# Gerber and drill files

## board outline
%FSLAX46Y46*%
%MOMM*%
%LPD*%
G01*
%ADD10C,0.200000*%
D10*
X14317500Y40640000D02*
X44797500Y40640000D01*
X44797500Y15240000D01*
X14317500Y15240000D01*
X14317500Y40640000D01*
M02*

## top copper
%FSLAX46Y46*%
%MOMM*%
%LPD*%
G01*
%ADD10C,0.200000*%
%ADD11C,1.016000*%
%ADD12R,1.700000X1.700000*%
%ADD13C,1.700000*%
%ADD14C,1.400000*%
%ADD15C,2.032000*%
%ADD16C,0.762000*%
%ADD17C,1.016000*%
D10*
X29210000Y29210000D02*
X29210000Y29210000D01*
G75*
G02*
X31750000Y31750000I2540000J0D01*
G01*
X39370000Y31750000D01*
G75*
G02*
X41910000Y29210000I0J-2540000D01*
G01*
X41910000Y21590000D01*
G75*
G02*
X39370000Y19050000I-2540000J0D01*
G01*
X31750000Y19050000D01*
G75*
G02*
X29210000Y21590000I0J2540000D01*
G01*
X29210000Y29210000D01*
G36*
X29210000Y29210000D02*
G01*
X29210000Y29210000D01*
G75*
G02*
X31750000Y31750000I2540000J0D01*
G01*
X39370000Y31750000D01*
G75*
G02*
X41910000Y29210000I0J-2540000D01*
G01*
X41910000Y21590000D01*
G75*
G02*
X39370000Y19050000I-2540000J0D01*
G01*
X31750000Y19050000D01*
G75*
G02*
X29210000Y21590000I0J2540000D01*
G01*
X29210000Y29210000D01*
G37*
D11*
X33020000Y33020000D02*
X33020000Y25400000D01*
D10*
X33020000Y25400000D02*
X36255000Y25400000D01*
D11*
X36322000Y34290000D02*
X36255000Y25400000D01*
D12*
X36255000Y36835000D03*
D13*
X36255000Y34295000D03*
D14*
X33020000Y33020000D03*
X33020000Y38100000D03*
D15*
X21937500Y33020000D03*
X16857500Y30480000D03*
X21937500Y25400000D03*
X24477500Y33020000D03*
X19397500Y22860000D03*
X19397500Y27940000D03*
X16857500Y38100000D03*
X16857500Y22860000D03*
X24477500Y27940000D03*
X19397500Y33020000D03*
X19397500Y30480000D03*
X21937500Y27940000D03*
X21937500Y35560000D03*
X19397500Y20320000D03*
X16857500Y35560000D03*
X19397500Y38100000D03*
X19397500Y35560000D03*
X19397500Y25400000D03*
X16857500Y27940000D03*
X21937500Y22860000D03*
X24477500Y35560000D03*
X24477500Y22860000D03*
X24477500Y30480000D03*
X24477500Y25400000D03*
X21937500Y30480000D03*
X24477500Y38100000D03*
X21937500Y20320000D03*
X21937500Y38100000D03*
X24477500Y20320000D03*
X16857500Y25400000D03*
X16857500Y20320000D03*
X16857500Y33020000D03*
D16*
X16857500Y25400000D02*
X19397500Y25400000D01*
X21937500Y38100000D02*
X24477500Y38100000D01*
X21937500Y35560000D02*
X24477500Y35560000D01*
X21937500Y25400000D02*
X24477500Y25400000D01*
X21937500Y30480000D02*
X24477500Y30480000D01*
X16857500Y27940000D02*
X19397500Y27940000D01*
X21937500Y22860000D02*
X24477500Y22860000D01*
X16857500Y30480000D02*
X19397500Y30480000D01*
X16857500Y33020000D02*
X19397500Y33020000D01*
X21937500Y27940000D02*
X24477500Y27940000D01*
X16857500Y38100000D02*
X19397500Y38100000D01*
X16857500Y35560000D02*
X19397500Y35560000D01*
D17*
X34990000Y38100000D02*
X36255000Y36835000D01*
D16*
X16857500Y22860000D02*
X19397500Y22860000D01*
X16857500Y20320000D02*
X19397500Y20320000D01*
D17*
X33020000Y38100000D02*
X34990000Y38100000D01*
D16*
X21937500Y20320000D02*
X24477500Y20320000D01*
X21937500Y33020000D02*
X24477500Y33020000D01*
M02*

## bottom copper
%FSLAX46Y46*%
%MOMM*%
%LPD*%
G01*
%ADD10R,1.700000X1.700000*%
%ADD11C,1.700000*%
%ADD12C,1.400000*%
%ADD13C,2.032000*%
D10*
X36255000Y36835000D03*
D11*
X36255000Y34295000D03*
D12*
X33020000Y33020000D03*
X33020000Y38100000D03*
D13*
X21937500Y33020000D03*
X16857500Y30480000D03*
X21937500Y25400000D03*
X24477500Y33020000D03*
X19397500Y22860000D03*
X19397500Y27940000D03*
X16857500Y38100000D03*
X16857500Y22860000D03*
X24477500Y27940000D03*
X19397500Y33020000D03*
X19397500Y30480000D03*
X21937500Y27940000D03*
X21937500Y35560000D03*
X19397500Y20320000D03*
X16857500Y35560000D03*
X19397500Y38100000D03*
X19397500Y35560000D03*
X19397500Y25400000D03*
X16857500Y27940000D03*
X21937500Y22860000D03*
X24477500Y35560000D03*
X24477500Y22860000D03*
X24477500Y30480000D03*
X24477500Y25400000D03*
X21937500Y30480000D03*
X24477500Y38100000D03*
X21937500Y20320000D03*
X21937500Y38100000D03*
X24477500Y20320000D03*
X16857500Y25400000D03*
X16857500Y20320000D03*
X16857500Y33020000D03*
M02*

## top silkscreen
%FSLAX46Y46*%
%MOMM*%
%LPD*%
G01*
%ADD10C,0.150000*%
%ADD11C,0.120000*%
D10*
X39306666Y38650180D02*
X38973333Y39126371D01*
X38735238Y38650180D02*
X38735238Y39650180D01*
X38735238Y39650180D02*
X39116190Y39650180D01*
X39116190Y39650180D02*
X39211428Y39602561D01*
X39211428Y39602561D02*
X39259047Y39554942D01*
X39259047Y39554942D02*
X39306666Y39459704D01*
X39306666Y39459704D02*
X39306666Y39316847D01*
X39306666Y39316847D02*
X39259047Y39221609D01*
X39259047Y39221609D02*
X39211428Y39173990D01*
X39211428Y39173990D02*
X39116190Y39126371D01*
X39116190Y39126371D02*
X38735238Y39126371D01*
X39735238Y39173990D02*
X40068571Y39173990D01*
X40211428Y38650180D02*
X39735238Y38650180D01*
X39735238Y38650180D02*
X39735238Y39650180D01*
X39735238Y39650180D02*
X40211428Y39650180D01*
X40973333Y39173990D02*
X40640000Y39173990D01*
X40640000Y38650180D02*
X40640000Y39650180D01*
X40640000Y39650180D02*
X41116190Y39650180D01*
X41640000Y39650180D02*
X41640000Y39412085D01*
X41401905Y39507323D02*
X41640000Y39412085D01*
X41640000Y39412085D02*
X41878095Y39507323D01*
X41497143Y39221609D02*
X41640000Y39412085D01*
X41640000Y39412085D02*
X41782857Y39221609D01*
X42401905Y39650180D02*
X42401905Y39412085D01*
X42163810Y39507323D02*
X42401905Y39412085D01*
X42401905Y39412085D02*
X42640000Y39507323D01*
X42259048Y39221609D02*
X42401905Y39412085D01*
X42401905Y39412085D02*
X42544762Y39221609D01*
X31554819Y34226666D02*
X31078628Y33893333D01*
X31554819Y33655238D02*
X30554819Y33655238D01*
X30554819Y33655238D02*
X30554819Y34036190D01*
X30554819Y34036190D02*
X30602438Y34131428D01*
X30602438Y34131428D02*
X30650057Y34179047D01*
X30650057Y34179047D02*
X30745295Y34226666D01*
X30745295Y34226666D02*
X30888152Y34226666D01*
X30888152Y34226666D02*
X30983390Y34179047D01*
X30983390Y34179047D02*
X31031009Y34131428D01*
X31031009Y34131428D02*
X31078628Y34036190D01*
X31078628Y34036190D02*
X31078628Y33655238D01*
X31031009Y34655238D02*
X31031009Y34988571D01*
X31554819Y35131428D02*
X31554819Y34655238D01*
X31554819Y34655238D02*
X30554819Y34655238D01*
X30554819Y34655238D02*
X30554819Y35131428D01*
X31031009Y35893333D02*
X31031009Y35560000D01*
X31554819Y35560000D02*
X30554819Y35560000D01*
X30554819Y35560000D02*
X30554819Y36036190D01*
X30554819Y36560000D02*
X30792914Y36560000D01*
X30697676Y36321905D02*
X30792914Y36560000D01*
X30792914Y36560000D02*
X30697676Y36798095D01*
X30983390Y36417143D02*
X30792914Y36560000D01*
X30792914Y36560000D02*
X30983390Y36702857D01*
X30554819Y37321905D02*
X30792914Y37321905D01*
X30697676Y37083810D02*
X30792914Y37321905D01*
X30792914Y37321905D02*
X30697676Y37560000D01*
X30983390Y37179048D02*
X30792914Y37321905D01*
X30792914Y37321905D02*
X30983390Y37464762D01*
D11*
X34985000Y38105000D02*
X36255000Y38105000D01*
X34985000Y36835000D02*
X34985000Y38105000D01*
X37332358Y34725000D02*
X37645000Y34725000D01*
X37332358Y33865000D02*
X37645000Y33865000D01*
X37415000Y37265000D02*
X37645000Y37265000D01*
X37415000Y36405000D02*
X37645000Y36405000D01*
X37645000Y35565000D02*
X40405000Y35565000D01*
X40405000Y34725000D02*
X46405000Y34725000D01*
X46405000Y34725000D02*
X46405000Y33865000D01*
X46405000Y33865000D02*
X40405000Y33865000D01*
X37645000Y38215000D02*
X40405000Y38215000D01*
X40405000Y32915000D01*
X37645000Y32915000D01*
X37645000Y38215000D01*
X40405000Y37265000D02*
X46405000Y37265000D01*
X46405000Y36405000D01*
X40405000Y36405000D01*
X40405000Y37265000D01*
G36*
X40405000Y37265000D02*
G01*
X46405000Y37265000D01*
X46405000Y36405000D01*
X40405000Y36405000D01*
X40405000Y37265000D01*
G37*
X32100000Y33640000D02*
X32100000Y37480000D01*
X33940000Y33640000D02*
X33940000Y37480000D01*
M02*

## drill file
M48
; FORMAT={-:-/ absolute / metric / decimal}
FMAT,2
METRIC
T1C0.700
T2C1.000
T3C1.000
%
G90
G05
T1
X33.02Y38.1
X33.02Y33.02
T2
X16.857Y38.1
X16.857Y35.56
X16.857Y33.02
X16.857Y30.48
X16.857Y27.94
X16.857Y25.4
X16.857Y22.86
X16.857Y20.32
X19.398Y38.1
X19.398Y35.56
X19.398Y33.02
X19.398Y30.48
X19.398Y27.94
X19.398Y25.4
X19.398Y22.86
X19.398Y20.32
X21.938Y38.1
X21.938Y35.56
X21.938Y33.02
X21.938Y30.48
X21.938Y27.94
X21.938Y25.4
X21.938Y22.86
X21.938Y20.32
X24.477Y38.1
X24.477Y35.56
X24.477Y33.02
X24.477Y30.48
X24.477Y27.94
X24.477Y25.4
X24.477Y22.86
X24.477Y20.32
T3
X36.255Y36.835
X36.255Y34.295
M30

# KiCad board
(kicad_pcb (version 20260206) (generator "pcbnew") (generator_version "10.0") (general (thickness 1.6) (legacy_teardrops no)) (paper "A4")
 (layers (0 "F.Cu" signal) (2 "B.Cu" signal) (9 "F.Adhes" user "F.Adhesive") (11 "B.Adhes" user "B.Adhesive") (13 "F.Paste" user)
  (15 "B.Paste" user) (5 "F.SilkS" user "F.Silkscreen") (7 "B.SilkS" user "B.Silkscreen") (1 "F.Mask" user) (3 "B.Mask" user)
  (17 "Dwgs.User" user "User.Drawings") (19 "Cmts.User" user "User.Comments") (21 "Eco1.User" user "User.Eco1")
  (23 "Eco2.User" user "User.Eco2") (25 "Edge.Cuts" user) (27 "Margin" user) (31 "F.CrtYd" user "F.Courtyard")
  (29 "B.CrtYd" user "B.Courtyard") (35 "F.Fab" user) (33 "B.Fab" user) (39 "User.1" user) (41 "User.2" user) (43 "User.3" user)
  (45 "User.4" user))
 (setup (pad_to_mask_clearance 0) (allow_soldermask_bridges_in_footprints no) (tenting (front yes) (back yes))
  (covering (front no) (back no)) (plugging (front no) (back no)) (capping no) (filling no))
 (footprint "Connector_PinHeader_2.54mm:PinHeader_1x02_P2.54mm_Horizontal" (layer "F.Cu") (at 36.255 -36.835)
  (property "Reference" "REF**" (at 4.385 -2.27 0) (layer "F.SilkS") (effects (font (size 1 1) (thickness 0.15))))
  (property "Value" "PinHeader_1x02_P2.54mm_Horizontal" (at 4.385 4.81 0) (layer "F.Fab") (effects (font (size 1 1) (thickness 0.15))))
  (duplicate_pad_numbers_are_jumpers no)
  (fp_line (start -1.27 -1.27) (end 0 -1.27) (stroke (width 0.12) (type solid)) (layer "F.SilkS"))
  (fp_line (start -1.27 0) (end -1.27 -1.27) (stroke (width 0.12) (type solid)) (layer "F.SilkS"))
  (fp_line (start 1.077358 2.11) (end 1.39 2.11) (stroke (width 0.12) (type solid)) (layer "F.SilkS"))
  (fp_line (start 1.077358 2.97) (end 1.39 2.97) (stroke (width 0.12) (type solid)) (layer "F.SilkS"))
  (fp_line (start 1.16 -0.43) (end 1.39 -0.43) (stroke (width 0.12) (type solid)) (layer "F.SilkS"))
  (fp_line (start 1.16 0.43) (end 1.39 0.43) (stroke (width 0.12) (type solid)) (layer "F.SilkS"))
  (fp_line (start 1.39 1.27) (end 4.15 1.27) (stroke (width 0.12) (type solid)) (layer "F.SilkS"))
  (fp_line (start 4.15 2.11) (end 10.15 2.11) (stroke (width 0.12) (type solid)) (layer "F.SilkS"))
  (fp_line (start 10.15 2.11) (end 10.15 2.97) (stroke (width 0.12) (type solid)) (layer "F.SilkS"))
  (fp_line (start 10.15 2.97) (end 4.15 2.97) (stroke (width 0.12) (type solid)) (layer "F.SilkS"))
  (fp_rect (start 1.39 -1.38) (end 4.15 3.92) (stroke (width 0.12) (type solid)) (fill no) (layer "F.SilkS"))
  (fp_rect (start 4.15 -0.43) (end 10.15 0.43) (stroke (width 0.12) (type solid)) (fill yes) (layer "F.SilkS"))
  (pad "1" thru_hole rect (at 0 0) (size 1.7 1.7) (drill 1) (layers "*.Cu" "*.Mask") (remove_unused_layers no))
  (pad "2" thru_hole circle (at 0 2.54) (size 1.7 1.7) (drill 1) (layers "*.Cu" "*.Mask") (remove_unused_layers no)))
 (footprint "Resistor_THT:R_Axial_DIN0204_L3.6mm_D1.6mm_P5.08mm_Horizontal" (layer "F.Cu") (at 33.02 -33.02 90)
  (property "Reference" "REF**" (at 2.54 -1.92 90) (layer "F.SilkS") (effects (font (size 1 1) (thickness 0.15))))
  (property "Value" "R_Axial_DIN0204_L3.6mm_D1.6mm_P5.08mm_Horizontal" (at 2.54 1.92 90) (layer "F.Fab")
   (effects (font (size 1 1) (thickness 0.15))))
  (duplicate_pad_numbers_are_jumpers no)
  (fp_line (start 0.62 -0.92) (end 4.46 -0.92) (stroke (width 0.12) (type solid)) (layer "F.SilkS"))
  (fp_line (start 0.62 0.92) (end 4.46 0.92) (stroke (width 0.12) (type solid)) (layer "F.SilkS"))
  (pad "1" thru_hole circle (at 0 0 90) (size 1.4 1.4) (drill 0.7) (layers "*.Cu" "*.Mask") (remove_unused_layers no))
  (pad "2" thru_hole circle (at 5.08 0 90) (size 1.4 1.4) (drill 0.7) (layers "*.Cu" "*.Mask") (remove_unused_layers no)))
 (gr_rect (start 29.21 -31.75) (end 41.91 -19.05) (radius 2.54) (stroke (width 0.2) (type default)) (fill yes) (layer "F.Cu"))
 (gr_line (start 33.02 -33.02) (end 33.02 -25.4) (stroke (width 1.016) (type default)) (layer "F.Cu"))
 (gr_line (start 33.02 -25.4) (end 36.255 -25.4) (stroke (width 0.2) (type default)) (layer "F.Cu"))
 (gr_line (start 36.322 -34.29) (end 36.255 -25.4) (stroke (width 1.016) (type default)) (layer "F.Cu"))
 (gr_rect (start 14.3175 -40.64) (end 44.7975 -15.24) (stroke (width 0.2) (type default)) (fill no) (layer "Edge.Cuts"))
 (segment (start 16.8575 -25.4) (end 19.3975 -25.4) (width 0.762) (layer "F.Cu") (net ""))
 (segment (start 21.9375 -38.1) (end 24.4775 -38.1) (width 0.762) (layer "F.Cu") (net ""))
 (segment (start 21.9375 -35.56) (end 24.4775 -35.56) (width 0.762) (layer "F.Cu") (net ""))
 (segment (start 21.9375 -25.4) (end 24.4775 -25.4) (width 0.762) (layer "F.Cu") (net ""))
 (segment (start 21.9375 -30.48) (end 24.4775 -30.48) (width 0.762) (layer "F.Cu") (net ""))
 (segment (start 16.8575 -27.94) (end 19.3975 -27.94) (width 0.762) (layer "F.Cu") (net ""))
 (segment (start 21.9375 -22.86) (end 24.4775 -22.86) (width 0.762) (layer "F.Cu") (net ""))
 (segment (start 16.8575 -30.48) (end 19.3975 -30.48) (width 0.762) (layer "F.Cu") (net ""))
 (segment (start 16.8575 -33.02) (end 19.3975 -33.02) (width 0.762) (layer "F.Cu") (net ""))
 (segment (start 21.9375 -27.94) (end 24.4775 -27.94) (width 0.762) (layer "F.Cu") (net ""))
 (segment (start 16.8575 -38.1) (end 19.3975 -38.1) (width 0.762) (layer "F.Cu") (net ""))
 (segment (start 16.8575 -35.56) (end 19.3975 -35.56) (width 0.762) (layer "F.Cu") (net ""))
 (segment (start 34.99 -38.1) (end 36.255 -36.835) (width 1.016) (layer "F.Cu") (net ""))
 (segment (start 16.8575 -22.86) (end 19.3975 -22.86) (width 0.762) (layer "F.Cu") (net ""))
 (segment (start 16.8575 -20.32) (end 19.3975 -20.32) (width 0.762) (layer "F.Cu") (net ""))
 (segment (start 33.02 -38.1) (end 34.99 -38.1) (width 1.016) (layer "F.Cu") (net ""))
 (segment (start 21.9375 -20.32) (end 24.4775 -20.32) (width 0.762) (layer "F.Cu") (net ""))
 (segment (start 21.9375 -33.02) (end 24.4775 -33.02) (width 0.762) (layer "F.Cu") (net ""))
 (via (at 21.9375 -33.02) (size 2.032) (drill 1) (layers "F.Cu" "B.Cu") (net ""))
 (via (at 16.8575 -30.48) (size 2.032) (drill 1) (layers "F.Cu" "B.Cu") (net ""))
 (via (at 21.9375 -25.4) (size 2.032) (drill 1) (layers "F.Cu" "B.Cu") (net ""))
 (via (at 24.4775 -33.02) (size 2.032) (drill 1) (layers "F.Cu" "B.Cu") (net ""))
 (via (at 19.3975 -22.86) (size 2.032) (drill 1) (layers "F.Cu" "B.Cu") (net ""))
 (via (at 19.3975 -27.94) (size 2.032) (drill 1) (layers "F.Cu" "B.Cu") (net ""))
 (via (at 16.8575 -38.1) (size 2.032) (drill 1) (layers "F.Cu" "B.Cu") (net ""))
 (via (at 16.8575 -22.86) (size 2.032) (drill 1) (layers "F.Cu" "B.Cu") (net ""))
 (via (at 24.4775 -27.94) (size 2.032) (drill 1) (layers "F.Cu" "B.Cu") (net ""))
 (via (at 19.3975 -33.02) (size 2.032) (drill 1) (layers "F.Cu" "B.Cu") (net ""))
 (via (at 19.3975 -30.48) (size 2.032) (drill 1) (layers "F.Cu" "B.Cu") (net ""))
 (via (at 21.9375 -27.94) (size 2.032) (drill 1) (layers "F.Cu" "B.Cu") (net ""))
 (via (at 21.9375 -35.56) (size 2.032) (drill 1) (layers "F.Cu" "B.Cu") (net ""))
 (via (at 19.3975 -20.32) (size 2.032) (drill 1) (layers "F.Cu" "B.Cu") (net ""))
 (via (at 16.8575 -35.56) (size 2.032) (drill 1) (layers "F.Cu" "B.Cu") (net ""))
 (via (at 19.3975 -38.1) (size 2.032) (drill 1) (layers "F.Cu" "B.Cu") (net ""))
 (via (at 19.3975 -35.56) (size 2.032) (drill 1) (layers "F.Cu" "B.Cu") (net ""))
 (via (at 19.3975 -25.4) (size 2.032) (drill 1) (layers "F.Cu" "B.Cu") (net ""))
 (via (at 16.8575 -27.94) (size 2.032) (drill 1) (layers "F.Cu" "B.Cu") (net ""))
 (via (at 21.9375 -22.86) (size 2.032) (drill 1) (layers "F.Cu" "B.Cu") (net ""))
 (via (at 24.4775 -35.56) (size 2.032) (drill 1) (layers "F.Cu" "B.Cu") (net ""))
 (via (at 24.4775 -22.86) (size 2.032) (drill 1) (layers "F.Cu" "B.Cu") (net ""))
 (via (at 24.4775 -30.48) (size 2.032) (drill 1) (layers "F.Cu" "B.Cu") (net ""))
 (via (at 24.4775 -25.4) (size 2.032) (drill 1) (layers "F.Cu" "B.Cu") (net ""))
 (via (at 21.9375 -30.48) (size 2.032) (drill 1) (layers "F.Cu" "B.Cu") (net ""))
 (via (at 24.4775 -38.1) (size 2.032) (drill 1) (layers "F.Cu" "B.Cu") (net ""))
 (via (at 21.9375 -20.32) (size 2.032) (drill 1) (layers "F.Cu" "B.Cu") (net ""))
 (via (at 21.9375 -38.1) (size 2.032) (drill 1) (layers "F.Cu" "B.Cu") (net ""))
 (via (at 24.4775 -20.32) (size 2.032) (drill 1) (layers "F.Cu" "B.Cu") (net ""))
 (via (at 16.8575 -25.4) (size 2.032) (drill 1) (layers "F.Cu" "B.Cu") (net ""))
 (via (at 16.8575 -20.32) (size 2.032) (drill 1) (layers "F.Cu" "B.Cu") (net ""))
 (via (at 16.8575 -33.02) (size 2.032) (drill 1) (layers "F.Cu" "B.Cu") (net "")))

